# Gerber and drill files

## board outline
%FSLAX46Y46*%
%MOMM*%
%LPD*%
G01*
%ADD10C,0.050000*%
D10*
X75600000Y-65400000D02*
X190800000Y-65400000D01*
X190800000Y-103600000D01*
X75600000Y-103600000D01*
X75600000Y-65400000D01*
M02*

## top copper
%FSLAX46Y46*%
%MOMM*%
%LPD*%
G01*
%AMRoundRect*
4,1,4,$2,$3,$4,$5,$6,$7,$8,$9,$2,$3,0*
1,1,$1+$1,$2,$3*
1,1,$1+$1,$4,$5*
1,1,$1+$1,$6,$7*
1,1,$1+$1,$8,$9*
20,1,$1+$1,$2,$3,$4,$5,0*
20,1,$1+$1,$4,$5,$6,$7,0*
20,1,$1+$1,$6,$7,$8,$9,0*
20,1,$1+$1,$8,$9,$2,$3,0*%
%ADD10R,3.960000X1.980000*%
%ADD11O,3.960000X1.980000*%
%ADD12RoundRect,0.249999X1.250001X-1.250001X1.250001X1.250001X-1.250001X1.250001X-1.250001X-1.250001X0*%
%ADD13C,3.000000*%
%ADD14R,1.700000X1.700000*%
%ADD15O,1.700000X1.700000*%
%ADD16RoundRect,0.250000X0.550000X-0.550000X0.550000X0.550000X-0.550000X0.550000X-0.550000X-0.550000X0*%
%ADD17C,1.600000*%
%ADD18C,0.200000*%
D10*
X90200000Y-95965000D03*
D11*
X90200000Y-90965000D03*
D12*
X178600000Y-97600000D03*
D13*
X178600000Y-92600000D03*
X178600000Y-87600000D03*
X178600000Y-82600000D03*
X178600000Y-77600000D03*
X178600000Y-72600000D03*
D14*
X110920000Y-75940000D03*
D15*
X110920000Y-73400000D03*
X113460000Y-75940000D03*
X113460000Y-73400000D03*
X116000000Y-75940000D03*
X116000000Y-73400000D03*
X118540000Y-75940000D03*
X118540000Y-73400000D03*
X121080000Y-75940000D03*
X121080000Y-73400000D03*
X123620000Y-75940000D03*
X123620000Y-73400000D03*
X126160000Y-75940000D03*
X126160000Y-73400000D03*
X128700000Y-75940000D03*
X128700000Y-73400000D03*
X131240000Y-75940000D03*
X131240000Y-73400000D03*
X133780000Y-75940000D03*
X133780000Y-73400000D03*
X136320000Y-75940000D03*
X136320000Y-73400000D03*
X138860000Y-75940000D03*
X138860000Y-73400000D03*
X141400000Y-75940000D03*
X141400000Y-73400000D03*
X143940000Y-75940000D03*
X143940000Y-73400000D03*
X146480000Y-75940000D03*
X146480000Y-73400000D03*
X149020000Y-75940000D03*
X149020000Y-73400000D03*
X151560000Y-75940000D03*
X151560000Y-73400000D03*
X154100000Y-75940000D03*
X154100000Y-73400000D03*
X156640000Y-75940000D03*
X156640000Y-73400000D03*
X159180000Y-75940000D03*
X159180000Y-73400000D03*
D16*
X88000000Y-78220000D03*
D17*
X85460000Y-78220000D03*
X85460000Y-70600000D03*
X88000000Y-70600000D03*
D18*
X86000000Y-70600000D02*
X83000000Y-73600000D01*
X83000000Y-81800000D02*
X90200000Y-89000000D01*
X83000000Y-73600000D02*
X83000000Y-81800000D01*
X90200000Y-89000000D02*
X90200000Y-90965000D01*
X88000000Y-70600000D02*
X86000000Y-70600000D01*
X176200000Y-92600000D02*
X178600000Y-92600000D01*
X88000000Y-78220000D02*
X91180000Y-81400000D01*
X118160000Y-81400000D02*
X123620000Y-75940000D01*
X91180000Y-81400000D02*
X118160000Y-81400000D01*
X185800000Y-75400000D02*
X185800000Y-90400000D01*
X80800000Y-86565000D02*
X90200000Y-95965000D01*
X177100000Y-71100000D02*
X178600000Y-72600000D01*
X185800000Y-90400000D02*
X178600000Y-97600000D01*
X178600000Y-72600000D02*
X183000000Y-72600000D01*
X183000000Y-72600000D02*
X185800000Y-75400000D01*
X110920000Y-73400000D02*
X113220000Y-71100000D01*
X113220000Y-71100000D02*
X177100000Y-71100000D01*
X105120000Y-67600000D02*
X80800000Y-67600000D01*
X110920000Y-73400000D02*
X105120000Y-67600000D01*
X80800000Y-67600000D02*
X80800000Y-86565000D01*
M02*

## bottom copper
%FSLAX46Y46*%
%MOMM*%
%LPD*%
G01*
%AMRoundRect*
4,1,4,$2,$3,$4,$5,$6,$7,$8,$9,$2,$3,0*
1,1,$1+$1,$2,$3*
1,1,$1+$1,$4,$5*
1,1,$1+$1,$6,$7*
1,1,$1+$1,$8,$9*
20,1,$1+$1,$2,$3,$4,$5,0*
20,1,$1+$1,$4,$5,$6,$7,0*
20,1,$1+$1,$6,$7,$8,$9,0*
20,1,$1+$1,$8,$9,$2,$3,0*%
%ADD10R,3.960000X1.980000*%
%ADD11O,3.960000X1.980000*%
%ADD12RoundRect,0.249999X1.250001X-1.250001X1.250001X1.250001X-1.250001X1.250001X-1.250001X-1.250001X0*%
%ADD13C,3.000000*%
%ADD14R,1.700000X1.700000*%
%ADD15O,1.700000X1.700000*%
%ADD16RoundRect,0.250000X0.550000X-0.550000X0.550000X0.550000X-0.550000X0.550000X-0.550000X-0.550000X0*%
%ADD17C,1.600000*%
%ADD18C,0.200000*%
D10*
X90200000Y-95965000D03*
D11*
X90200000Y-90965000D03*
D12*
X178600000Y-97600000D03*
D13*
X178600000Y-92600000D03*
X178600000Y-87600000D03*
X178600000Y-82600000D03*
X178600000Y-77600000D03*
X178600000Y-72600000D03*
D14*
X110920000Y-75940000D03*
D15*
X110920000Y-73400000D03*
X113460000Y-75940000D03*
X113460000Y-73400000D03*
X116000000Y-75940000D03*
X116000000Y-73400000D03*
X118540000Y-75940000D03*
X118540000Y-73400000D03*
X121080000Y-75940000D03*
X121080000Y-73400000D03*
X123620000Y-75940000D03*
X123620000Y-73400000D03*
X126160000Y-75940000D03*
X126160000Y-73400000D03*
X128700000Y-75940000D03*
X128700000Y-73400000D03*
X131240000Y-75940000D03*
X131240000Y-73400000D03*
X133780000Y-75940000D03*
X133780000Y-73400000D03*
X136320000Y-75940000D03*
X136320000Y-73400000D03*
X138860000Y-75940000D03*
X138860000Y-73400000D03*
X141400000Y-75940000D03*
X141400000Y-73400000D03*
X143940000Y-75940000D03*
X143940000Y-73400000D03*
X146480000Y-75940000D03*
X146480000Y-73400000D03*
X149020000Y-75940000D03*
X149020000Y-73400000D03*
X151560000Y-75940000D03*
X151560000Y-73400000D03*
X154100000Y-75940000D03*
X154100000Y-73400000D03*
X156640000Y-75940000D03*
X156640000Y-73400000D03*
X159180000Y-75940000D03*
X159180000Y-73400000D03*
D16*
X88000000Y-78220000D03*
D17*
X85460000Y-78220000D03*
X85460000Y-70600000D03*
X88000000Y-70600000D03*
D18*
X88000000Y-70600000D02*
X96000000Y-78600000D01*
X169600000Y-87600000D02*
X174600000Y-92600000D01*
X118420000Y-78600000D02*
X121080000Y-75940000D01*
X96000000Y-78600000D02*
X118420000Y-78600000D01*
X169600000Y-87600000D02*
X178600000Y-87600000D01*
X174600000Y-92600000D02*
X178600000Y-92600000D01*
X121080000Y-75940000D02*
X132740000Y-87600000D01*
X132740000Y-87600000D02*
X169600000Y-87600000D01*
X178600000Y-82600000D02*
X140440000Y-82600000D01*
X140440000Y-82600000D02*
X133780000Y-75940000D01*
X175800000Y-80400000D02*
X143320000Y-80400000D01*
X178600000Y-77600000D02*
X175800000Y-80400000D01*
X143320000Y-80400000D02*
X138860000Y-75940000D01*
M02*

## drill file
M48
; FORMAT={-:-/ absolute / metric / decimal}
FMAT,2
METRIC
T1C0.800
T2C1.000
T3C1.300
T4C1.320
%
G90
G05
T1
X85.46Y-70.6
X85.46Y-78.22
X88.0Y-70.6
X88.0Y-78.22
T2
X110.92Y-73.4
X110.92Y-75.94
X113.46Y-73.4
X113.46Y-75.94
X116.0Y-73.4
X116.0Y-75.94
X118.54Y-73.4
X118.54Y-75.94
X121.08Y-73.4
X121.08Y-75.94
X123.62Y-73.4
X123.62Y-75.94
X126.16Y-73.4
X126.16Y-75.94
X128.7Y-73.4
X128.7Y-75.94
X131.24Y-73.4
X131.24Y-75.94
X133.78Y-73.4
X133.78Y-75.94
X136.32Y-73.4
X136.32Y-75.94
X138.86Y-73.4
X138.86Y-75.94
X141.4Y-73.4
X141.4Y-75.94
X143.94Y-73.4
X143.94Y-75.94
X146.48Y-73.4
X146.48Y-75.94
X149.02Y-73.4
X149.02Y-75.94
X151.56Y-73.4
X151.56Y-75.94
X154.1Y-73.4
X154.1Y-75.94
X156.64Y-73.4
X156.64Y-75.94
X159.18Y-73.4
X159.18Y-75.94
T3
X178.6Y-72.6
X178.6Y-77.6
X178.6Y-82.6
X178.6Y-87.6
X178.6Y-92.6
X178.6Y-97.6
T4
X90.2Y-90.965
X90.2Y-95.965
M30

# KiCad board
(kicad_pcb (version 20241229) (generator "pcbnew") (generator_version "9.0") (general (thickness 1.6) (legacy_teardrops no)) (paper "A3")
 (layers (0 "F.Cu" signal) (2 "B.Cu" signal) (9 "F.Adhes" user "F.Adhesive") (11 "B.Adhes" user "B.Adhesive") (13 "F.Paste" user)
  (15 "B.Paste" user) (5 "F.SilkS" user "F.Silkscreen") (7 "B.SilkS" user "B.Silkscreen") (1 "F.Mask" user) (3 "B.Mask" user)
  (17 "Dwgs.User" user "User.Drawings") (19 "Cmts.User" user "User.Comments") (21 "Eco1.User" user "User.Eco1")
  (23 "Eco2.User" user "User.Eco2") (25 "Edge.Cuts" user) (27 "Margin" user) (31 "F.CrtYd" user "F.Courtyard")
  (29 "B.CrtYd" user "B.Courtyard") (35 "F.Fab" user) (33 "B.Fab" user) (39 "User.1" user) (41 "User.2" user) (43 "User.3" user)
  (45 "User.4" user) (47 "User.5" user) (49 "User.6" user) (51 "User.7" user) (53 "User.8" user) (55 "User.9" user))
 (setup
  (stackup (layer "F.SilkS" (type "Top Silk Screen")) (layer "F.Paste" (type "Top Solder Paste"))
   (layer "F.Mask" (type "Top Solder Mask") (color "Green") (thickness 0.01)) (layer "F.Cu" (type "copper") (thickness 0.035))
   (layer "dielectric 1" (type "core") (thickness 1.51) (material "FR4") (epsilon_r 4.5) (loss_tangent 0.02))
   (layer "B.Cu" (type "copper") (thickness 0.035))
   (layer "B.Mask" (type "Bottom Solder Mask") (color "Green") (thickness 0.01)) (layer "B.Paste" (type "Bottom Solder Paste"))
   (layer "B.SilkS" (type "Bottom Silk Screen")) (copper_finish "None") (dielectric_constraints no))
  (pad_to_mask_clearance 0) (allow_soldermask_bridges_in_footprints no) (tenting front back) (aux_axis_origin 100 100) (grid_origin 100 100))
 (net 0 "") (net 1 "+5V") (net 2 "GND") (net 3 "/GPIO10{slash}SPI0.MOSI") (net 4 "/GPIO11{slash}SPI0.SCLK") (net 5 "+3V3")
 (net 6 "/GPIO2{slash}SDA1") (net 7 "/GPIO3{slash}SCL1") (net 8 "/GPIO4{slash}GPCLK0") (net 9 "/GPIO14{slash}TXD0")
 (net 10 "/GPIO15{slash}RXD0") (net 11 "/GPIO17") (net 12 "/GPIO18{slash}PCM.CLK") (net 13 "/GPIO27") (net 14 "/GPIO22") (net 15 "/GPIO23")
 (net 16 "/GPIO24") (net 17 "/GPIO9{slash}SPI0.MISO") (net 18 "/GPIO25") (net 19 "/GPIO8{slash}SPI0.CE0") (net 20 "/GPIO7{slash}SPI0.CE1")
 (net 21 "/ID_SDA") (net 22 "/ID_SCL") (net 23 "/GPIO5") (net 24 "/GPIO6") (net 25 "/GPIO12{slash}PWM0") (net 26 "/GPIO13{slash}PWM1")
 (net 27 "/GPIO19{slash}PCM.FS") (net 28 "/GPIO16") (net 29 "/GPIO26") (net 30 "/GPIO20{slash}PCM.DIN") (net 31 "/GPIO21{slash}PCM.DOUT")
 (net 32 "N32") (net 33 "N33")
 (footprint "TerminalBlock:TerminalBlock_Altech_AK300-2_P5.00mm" (layer "F.Cu") (at 90.2 95.965 90)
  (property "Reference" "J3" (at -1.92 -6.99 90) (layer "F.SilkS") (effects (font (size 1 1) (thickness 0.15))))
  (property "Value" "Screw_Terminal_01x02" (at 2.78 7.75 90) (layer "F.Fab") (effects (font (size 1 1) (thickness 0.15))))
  (pad "1" thru_hole rect (at 0 0 90) (size 1.98 3.96) (drill 1.32) (layers "*.Cu" "*.Mask") (remove_unused_layers no) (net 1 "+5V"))
  (pad "2" thru_hole oval (at 5 0 90) (size 1.98 3.96) (drill 1.32) (layers "*.Cu" "*.Mask") (remove_unused_layers no) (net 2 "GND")))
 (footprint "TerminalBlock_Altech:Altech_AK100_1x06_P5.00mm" (layer "F.Cu") (at 178.6 97.6 90)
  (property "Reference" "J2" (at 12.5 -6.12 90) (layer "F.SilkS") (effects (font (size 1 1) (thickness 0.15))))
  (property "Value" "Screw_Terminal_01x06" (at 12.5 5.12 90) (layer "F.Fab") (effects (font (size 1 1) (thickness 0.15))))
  (pad "1" thru_hole roundrect (at 0 0 90) (size 3 3) (drill 1.3) (layers "*.Cu" "*.Mask") (remove_unused_layers no)
   (roundrect_rratio 0.083333) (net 1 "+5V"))
  (pad "2" thru_hole circle (at 5 0 90) (size 3 3) (drill 1.3) (layers "*.Cu" "*.Mask") (remove_unused_layers no) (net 2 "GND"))
  (pad "3" thru_hole circle (at 10 0 90) (size 3 3) (drill 1.3) (layers "*.Cu" "*.Mask") (remove_unused_layers no) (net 2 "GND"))
  (pad "4" thru_hole circle (at 15 0 90) (size 3 3) (drill 1.3) (layers "*.Cu" "*.Mask") (remove_unused_layers no)
   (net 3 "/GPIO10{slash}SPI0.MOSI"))
  (pad "5" thru_hole circle (at 20 0 90) (size 3 3) (drill 1.3) (layers "*.Cu" "*.Mask") (remove_unused_layers no)
   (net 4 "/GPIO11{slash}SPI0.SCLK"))
  (pad "6" thru_hole circle (at 25 0 90) (size 3 3) (drill 1.3) (layers "*.Cu" "*.Mask") (remove_unused_layers no) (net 1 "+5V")))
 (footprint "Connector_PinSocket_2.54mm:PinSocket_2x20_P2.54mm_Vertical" (layer "B.Cu") (at 110.92 75.94 -90)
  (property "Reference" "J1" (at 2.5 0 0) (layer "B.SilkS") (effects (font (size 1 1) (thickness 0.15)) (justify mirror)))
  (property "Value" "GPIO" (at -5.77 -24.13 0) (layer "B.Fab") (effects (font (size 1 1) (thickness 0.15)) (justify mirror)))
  (pad "1" thru_hole rect (at 0 0 270) (size 1.7 1.7) (drill 1) (layers "*.Cu" "*.Mask") (remove_unused_layers no) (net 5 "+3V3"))
  (pad "2" thru_hole oval (at -2.54 0 270) (size 1.7 1.7) (drill 1) (layers "*.Cu" "*.Mask") (remove_unused_layers no) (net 1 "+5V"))
  (pad "3" thru_hole oval (at 0 -2.54 270) (size 1.7 1.7) (drill 1) (layers "*.Cu" "*.Mask") (remove_unused_layers no)
   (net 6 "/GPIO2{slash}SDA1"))
  (pad "4" thru_hole oval (at -2.54 -2.54 270) (size 1.7 1.7) (drill 1) (layers "*.Cu" "*.Mask") (remove_unused_layers no) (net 1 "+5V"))
  (pad "5" thru_hole oval (at 0 -5.08 270) (size 1.7 1.7) (drill 1) (layers "*.Cu" "*.Mask") (remove_unused_layers no)
   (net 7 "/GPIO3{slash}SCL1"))
  (pad "6" thru_hole oval (at -2.54 -5.08 270) (size 1.7 1.7) (drill 1) (layers "*.Cu" "*.Mask") (remove_unused_layers no) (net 2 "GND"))
  (pad "7" thru_hole oval (at 0 -7.62 270) (size 1.7 1.7) (drill 1) (layers "*.Cu" "*.Mask") (remove_unused_layers no)
   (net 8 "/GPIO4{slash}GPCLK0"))
  (pad "8" thru_hole oval (at -2.54 -7.62 270) (size 1.7 1.7) (drill 1) (layers "*.Cu" "*.Mask") (remove_unused_layers no)
   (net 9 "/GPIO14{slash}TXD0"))
  (pad "9" thru_hole oval (at 0 -10.16 270) (size 1.7 1.7) (drill 1) (layers "*.Cu" "*.Mask") (remove_unused_layers no) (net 2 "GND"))
  (pad "10" thru_hole oval (at -2.54 -10.16 270) (size 1.7 1.7) (drill 1) (layers "*.Cu" "*.Mask") (remove_unused_layers no)
   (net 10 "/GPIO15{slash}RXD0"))
  (pad "11" thru_hole oval (at 0 -12.7 270) (size 1.7 1.7) (drill 1) (layers "*.Cu" "*.Mask") (remove_unused_layers no) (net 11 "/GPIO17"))
  (pad "12" thru_hole oval (at -2.54 -12.7 270) (size 1.7 1.7) (drill 1) (layers "*.Cu" "*.Mask") (remove_unused_layers no)
   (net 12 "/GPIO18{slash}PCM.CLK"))
  (pad "13" thru_hole oval (at 0 -15.24 270) (size 1.7 1.7) (drill 1) (layers "*.Cu" "*.Mask") (remove_unused_layers no) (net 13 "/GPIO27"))
  (pad "14" thru_hole oval (at -2.54 -15.24 270) (size 1.7 1.7) (drill 1) (layers "*.Cu" "*.Mask") (remove_unused_layers no) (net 2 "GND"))
  (pad "15" thru_hole oval (at 0 -17.78 270) (size 1.7 1.7) (drill 1) (layers "*.Cu" "*.Mask") (remove_unused_layers no) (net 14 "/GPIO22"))
  (pad "16" thru_hole oval (at -2.54 -17.78 270) (size 1.7 1.7) (drill 1) (layers "*.Cu" "*.Mask") (remove_unused_layers no)
   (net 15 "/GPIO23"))
  (pad "17" thru_hole oval (at 0 -20.32 270) (size 1.7 1.7) (drill 1) (layers "*.Cu" "*.Mask") (remove_unused_layers no) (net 5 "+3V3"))
  (pad "18" thru_hole oval (at -2.54 -20.32 270) (size 1.7 1.7) (drill 1) (layers "*.Cu" "*.Mask") (remove_unused_layers no)
   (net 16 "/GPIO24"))
  (pad "19" thru_hole oval (at 0 -22.86 270) (size 1.7 1.7) (drill 1) (layers "*.Cu" "*.Mask") (remove_unused_layers no)
   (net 3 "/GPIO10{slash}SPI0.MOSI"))
  (pad "20" thru_hole oval (at -2.54 -22.86 270) (size 1.7 1.7) (drill 1) (layers "*.Cu" "*.Mask") (remove_unused_layers no) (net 2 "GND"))
  (pad "21" thru_hole oval (at 0 -25.4 270) (size 1.7 1.7) (drill 1) (layers "*.Cu" "*.Mask") (remove_unused_layers no)
   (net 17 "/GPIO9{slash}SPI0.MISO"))
  (pad "22" thru_hole oval (at -2.54 -25.4 270) (size 1.7 1.7) (drill 1) (layers "*.Cu" "*.Mask") (remove_unused_layers no)
   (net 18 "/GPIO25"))
  (pad "23" thru_hole oval (at 0 -27.94 270) (size 1.7 1.7) (drill 1) (layers "*.Cu" "*.Mask") (remove_unused_layers no)
   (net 4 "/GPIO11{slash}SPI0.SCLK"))
  (pad "24" thru_hole oval (at -2.54 -27.94 270) (size 1.7 1.7) (drill 1) (layers "*.Cu" "*.Mask") (remove_unused_layers no)
   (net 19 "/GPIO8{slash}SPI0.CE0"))
  (pad "25" thru_hole oval (at 0 -30.48 270) (size 1.7 1.7) (drill 1) (layers "*.Cu" "*.Mask") (remove_unused_layers no) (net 2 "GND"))
  (pad "26" thru_hole oval (at -2.54 -30.48 270) (size 1.7 1.7) (drill 1) (layers "*.Cu" "*.Mask") (remove_unused_layers no)
   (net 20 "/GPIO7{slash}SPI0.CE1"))
  (pad "27" thru_hole oval (at 0 -33.02 270) (size 1.7 1.7) (drill 1) (layers "*.Cu" "*.Mask") (remove_unused_layers no) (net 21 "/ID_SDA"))
  (pad "28" thru_hole oval (at -2.54 -33.02 270) (size 1.7 1.7) (drill 1) (layers "*.Cu" "*.Mask") (remove_unused_layers no)
   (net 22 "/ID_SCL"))
  (pad "29" thru_hole oval (at 0 -35.56 270) (size 1.7 1.7) (drill 1) (layers "*.Cu" "*.Mask") (remove_unused_layers no) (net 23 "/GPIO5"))
  (pad "30" thru_hole oval (at -2.54 -35.56 270) (size 1.7 1.7) (drill 1) (layers "*.Cu" "*.Mask") (remove_unused_layers no) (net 2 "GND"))
  (pad "31" thru_hole oval (at 0 -38.1 270) (size 1.7 1.7) (drill 1) (layers "*.Cu" "*.Mask") (remove_unused_layers no) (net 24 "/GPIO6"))
  (pad "32" thru_hole oval (at -2.54 -38.1 270) (size 1.7 1.7) (drill 1) (layers "*.Cu" "*.Mask") (remove_unused_layers no)
   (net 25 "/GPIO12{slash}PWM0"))
  (pad "33" thru_hole oval (at 0 -40.64 270) (size 1.7 1.7) (drill 1) (layers "*.Cu" "*.Mask") (remove_unused_layers no)
   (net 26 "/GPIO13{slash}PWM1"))
  (pad "34" thru_hole oval (at -2.54 -40.64 270) (size 1.7 1.7) (drill 1) (layers "*.Cu" "*.Mask") (remove_unused_layers no) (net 2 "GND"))
  (pad "35" thru_hole oval (at 0 -43.18 270) (size 1.7 1.7) (drill 1) (layers "*.Cu" "*.Mask") (remove_unused_layers no)
   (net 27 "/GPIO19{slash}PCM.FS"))
  (pad "36" thru_hole oval (at -2.54 -43.18 270) (size 1.7 1.7) (drill 1) (layers "*.Cu" "*.Mask") (remove_unused_layers no)
   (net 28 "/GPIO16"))
  (pad "37" thru_hole oval (at 0 -45.72 270) (size 1.7 1.7) (drill 1) (layers "*.Cu" "*.Mask") (remove_unused_layers no) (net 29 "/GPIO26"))
  (pad "38" thru_hole oval (at -2.54 -45.72 270) (size 1.7 1.7) (drill 1) (layers "*.Cu" "*.Mask") (remove_unused_layers no)
   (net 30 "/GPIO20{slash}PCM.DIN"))
  (pad "39" thru_hole oval (at 0 -48.26 270) (size 1.7 1.7) (drill 1) (layers "*.Cu" "*.Mask") (remove_unused_layers no) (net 2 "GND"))
  (pad "40" thru_hole oval (at -2.54 -48.26 270) (size 1.7 1.7) (drill 1) (layers "*.Cu" "*.Mask") (remove_unused_layers no)
   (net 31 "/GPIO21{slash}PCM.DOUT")))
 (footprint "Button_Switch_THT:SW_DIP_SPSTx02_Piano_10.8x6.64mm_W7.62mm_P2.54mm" (layer "B.Cu") (at 88 78.22 90)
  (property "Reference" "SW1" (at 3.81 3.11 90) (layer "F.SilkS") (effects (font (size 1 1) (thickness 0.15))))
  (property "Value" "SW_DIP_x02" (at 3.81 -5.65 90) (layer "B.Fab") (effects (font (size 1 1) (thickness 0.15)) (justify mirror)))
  (pad "1" thru_hole roundrect (at 0 0 90) (size 1.6 1.6) (drill 0.8) (layers "*.Cu" "*.Mask") (remove_unused_layers no)
   (roundrect_rratio 0.15625) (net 11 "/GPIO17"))
  (pad "2" thru_hole circle (at 0 -2.54 90) (size 1.6 1.6) (drill 0.8) (layers "*.Cu" "*.Mask") (remove_unused_layers no) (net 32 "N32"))
  (pad "3" thru_hole circle (at 7.62 -2.54 90) (size 1.6 1.6) (drill 0.8) (layers "*.Cu" "*.Mask") (remove_unused_layers no) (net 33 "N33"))
  (pad "4" thru_hole circle (at 7.62 0 90) (size 1.6 1.6) (drill 0.8) (layers "*.Cu" "*.Mask") (remove_unused_layers no) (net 2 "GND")))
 (gr_rect (start 75.6 65.4) (end 190.8 103.6) (stroke (width 0.05) (type default)) (fill no) (layer "Edge.Cuts"))
 (segment (start 86 70.6) (end 83 73.6) (width 0.2) (layer "F.Cu") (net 2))
 (segment (start 83 81.8) (end 90.2 89) (width 0.2) (layer "F.Cu") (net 2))
 (segment (start 83 73.6) (end 83 81.8) (width 0.2) (layer "F.Cu") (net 2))
 (segment (start 90.2 89) (end 90.2 90.965) (width 0.2) (layer "F.Cu") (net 2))
 (segment (start 88 70.6) (end 86 70.6) (width 0.2) (layer "F.Cu") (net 2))
 (segment (start 176.2 92.6) (end 178.6 92.6) (width 0.2) (layer "F.Cu") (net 2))
 (segment (start 88 70.6) (end 96 78.6) (width 0.2) (layer "B.Cu") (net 2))
 (segment (start 169.6 87.6) (end 174.6 92.6) (width 0.2) (layer "B.Cu") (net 2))
 (segment (start 118.42 78.6) (end 121.08 75.94) (width 0.2) (layer "B.Cu") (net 2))
 (segment (start 96 78.6) (end 118.42 78.6) (width 0.2) (layer "B.Cu") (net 2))
 (segment (start 169.6 87.6) (end 178.6 87.6) (width 0.2) (layer "B.Cu") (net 2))
 (segment (start 174.6 92.6) (end 178.6 92.6) (width 0.2) (layer "B.Cu") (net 2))
 (segment (start 121.08 75.94) (end 132.74 87.6) (width 0.2) (layer "B.Cu") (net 2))
 (segment (start 132.74 87.6) (end 169.6 87.6) (width 0.2) (layer "B.Cu") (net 2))
 (segment (start 88 78.22) (end 91.18 81.4) (width 0.2) (layer "F.Cu") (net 11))
 (segment (start 118.16 81.4) (end 123.62 75.94) (width 0.2) (layer "F.Cu") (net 11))
 (segment (start 91.18 81.4) (end 118.16 81.4) (width 0.2) (layer "F.Cu") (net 11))
 (segment (start 178.6 82.6) (end 140.44 82.6) (width 0.2) (layer "B.Cu") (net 3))
 (segment (start 140.44 82.6) (end 133.78 75.94) (width 0.2) (layer "B.Cu") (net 3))
 (segment (start 175.8 80.4) (end 143.32 80.4) (width 0.2) (layer "B.Cu") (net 4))
 (segment (start 178.6 77.6) (end 175.8 80.4) (width 0.2) (layer "B.Cu") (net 4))
 (segment (start 143.32 80.4) (end 138.86 75.94) (width 0.2) (layer "B.Cu") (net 4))
 (segment (start 185.8 75.4) (end 185.8 90.4) (width 0.2) (layer "F.Cu") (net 1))
 (segment (start 80.8 86.565) (end 90.2 95.965) (width 0.2) (layer "F.Cu") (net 1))
 (segment (start 177.1 71.1) (end 178.6 72.6) (width 0.2) (layer "F.Cu") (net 1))
 (segment (start 185.8 90.4) (end 178.6 97.6) (width 0.2) (layer "F.Cu") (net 1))
 (segment (start 178.6 72.6) (end 183 72.6) (width 0.2) (layer "F.Cu") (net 1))
 (segment (start 183 72.6) (end 185.8 75.4) (width 0.2) (layer "F.Cu") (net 1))
 (segment (start 110.92 73.4) (end 113.22 71.1) (width 0.2) (layer "F.Cu") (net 1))
 (segment (start 113.22 71.1) (end 177.1 71.1) (width 0.2) (layer "F.Cu") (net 1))
 (segment (start 105.12 67.6) (end 80.8 67.6) (width 0.2) (layer "F.Cu") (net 1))
 (segment (start 110.92 73.4) (end 105.12 67.6) (width 0.2) (layer "F.Cu") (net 1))
 (segment (start 80.8 67.6) (end 80.8 86.565) (width 0.2) (layer "F.Cu") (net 1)))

